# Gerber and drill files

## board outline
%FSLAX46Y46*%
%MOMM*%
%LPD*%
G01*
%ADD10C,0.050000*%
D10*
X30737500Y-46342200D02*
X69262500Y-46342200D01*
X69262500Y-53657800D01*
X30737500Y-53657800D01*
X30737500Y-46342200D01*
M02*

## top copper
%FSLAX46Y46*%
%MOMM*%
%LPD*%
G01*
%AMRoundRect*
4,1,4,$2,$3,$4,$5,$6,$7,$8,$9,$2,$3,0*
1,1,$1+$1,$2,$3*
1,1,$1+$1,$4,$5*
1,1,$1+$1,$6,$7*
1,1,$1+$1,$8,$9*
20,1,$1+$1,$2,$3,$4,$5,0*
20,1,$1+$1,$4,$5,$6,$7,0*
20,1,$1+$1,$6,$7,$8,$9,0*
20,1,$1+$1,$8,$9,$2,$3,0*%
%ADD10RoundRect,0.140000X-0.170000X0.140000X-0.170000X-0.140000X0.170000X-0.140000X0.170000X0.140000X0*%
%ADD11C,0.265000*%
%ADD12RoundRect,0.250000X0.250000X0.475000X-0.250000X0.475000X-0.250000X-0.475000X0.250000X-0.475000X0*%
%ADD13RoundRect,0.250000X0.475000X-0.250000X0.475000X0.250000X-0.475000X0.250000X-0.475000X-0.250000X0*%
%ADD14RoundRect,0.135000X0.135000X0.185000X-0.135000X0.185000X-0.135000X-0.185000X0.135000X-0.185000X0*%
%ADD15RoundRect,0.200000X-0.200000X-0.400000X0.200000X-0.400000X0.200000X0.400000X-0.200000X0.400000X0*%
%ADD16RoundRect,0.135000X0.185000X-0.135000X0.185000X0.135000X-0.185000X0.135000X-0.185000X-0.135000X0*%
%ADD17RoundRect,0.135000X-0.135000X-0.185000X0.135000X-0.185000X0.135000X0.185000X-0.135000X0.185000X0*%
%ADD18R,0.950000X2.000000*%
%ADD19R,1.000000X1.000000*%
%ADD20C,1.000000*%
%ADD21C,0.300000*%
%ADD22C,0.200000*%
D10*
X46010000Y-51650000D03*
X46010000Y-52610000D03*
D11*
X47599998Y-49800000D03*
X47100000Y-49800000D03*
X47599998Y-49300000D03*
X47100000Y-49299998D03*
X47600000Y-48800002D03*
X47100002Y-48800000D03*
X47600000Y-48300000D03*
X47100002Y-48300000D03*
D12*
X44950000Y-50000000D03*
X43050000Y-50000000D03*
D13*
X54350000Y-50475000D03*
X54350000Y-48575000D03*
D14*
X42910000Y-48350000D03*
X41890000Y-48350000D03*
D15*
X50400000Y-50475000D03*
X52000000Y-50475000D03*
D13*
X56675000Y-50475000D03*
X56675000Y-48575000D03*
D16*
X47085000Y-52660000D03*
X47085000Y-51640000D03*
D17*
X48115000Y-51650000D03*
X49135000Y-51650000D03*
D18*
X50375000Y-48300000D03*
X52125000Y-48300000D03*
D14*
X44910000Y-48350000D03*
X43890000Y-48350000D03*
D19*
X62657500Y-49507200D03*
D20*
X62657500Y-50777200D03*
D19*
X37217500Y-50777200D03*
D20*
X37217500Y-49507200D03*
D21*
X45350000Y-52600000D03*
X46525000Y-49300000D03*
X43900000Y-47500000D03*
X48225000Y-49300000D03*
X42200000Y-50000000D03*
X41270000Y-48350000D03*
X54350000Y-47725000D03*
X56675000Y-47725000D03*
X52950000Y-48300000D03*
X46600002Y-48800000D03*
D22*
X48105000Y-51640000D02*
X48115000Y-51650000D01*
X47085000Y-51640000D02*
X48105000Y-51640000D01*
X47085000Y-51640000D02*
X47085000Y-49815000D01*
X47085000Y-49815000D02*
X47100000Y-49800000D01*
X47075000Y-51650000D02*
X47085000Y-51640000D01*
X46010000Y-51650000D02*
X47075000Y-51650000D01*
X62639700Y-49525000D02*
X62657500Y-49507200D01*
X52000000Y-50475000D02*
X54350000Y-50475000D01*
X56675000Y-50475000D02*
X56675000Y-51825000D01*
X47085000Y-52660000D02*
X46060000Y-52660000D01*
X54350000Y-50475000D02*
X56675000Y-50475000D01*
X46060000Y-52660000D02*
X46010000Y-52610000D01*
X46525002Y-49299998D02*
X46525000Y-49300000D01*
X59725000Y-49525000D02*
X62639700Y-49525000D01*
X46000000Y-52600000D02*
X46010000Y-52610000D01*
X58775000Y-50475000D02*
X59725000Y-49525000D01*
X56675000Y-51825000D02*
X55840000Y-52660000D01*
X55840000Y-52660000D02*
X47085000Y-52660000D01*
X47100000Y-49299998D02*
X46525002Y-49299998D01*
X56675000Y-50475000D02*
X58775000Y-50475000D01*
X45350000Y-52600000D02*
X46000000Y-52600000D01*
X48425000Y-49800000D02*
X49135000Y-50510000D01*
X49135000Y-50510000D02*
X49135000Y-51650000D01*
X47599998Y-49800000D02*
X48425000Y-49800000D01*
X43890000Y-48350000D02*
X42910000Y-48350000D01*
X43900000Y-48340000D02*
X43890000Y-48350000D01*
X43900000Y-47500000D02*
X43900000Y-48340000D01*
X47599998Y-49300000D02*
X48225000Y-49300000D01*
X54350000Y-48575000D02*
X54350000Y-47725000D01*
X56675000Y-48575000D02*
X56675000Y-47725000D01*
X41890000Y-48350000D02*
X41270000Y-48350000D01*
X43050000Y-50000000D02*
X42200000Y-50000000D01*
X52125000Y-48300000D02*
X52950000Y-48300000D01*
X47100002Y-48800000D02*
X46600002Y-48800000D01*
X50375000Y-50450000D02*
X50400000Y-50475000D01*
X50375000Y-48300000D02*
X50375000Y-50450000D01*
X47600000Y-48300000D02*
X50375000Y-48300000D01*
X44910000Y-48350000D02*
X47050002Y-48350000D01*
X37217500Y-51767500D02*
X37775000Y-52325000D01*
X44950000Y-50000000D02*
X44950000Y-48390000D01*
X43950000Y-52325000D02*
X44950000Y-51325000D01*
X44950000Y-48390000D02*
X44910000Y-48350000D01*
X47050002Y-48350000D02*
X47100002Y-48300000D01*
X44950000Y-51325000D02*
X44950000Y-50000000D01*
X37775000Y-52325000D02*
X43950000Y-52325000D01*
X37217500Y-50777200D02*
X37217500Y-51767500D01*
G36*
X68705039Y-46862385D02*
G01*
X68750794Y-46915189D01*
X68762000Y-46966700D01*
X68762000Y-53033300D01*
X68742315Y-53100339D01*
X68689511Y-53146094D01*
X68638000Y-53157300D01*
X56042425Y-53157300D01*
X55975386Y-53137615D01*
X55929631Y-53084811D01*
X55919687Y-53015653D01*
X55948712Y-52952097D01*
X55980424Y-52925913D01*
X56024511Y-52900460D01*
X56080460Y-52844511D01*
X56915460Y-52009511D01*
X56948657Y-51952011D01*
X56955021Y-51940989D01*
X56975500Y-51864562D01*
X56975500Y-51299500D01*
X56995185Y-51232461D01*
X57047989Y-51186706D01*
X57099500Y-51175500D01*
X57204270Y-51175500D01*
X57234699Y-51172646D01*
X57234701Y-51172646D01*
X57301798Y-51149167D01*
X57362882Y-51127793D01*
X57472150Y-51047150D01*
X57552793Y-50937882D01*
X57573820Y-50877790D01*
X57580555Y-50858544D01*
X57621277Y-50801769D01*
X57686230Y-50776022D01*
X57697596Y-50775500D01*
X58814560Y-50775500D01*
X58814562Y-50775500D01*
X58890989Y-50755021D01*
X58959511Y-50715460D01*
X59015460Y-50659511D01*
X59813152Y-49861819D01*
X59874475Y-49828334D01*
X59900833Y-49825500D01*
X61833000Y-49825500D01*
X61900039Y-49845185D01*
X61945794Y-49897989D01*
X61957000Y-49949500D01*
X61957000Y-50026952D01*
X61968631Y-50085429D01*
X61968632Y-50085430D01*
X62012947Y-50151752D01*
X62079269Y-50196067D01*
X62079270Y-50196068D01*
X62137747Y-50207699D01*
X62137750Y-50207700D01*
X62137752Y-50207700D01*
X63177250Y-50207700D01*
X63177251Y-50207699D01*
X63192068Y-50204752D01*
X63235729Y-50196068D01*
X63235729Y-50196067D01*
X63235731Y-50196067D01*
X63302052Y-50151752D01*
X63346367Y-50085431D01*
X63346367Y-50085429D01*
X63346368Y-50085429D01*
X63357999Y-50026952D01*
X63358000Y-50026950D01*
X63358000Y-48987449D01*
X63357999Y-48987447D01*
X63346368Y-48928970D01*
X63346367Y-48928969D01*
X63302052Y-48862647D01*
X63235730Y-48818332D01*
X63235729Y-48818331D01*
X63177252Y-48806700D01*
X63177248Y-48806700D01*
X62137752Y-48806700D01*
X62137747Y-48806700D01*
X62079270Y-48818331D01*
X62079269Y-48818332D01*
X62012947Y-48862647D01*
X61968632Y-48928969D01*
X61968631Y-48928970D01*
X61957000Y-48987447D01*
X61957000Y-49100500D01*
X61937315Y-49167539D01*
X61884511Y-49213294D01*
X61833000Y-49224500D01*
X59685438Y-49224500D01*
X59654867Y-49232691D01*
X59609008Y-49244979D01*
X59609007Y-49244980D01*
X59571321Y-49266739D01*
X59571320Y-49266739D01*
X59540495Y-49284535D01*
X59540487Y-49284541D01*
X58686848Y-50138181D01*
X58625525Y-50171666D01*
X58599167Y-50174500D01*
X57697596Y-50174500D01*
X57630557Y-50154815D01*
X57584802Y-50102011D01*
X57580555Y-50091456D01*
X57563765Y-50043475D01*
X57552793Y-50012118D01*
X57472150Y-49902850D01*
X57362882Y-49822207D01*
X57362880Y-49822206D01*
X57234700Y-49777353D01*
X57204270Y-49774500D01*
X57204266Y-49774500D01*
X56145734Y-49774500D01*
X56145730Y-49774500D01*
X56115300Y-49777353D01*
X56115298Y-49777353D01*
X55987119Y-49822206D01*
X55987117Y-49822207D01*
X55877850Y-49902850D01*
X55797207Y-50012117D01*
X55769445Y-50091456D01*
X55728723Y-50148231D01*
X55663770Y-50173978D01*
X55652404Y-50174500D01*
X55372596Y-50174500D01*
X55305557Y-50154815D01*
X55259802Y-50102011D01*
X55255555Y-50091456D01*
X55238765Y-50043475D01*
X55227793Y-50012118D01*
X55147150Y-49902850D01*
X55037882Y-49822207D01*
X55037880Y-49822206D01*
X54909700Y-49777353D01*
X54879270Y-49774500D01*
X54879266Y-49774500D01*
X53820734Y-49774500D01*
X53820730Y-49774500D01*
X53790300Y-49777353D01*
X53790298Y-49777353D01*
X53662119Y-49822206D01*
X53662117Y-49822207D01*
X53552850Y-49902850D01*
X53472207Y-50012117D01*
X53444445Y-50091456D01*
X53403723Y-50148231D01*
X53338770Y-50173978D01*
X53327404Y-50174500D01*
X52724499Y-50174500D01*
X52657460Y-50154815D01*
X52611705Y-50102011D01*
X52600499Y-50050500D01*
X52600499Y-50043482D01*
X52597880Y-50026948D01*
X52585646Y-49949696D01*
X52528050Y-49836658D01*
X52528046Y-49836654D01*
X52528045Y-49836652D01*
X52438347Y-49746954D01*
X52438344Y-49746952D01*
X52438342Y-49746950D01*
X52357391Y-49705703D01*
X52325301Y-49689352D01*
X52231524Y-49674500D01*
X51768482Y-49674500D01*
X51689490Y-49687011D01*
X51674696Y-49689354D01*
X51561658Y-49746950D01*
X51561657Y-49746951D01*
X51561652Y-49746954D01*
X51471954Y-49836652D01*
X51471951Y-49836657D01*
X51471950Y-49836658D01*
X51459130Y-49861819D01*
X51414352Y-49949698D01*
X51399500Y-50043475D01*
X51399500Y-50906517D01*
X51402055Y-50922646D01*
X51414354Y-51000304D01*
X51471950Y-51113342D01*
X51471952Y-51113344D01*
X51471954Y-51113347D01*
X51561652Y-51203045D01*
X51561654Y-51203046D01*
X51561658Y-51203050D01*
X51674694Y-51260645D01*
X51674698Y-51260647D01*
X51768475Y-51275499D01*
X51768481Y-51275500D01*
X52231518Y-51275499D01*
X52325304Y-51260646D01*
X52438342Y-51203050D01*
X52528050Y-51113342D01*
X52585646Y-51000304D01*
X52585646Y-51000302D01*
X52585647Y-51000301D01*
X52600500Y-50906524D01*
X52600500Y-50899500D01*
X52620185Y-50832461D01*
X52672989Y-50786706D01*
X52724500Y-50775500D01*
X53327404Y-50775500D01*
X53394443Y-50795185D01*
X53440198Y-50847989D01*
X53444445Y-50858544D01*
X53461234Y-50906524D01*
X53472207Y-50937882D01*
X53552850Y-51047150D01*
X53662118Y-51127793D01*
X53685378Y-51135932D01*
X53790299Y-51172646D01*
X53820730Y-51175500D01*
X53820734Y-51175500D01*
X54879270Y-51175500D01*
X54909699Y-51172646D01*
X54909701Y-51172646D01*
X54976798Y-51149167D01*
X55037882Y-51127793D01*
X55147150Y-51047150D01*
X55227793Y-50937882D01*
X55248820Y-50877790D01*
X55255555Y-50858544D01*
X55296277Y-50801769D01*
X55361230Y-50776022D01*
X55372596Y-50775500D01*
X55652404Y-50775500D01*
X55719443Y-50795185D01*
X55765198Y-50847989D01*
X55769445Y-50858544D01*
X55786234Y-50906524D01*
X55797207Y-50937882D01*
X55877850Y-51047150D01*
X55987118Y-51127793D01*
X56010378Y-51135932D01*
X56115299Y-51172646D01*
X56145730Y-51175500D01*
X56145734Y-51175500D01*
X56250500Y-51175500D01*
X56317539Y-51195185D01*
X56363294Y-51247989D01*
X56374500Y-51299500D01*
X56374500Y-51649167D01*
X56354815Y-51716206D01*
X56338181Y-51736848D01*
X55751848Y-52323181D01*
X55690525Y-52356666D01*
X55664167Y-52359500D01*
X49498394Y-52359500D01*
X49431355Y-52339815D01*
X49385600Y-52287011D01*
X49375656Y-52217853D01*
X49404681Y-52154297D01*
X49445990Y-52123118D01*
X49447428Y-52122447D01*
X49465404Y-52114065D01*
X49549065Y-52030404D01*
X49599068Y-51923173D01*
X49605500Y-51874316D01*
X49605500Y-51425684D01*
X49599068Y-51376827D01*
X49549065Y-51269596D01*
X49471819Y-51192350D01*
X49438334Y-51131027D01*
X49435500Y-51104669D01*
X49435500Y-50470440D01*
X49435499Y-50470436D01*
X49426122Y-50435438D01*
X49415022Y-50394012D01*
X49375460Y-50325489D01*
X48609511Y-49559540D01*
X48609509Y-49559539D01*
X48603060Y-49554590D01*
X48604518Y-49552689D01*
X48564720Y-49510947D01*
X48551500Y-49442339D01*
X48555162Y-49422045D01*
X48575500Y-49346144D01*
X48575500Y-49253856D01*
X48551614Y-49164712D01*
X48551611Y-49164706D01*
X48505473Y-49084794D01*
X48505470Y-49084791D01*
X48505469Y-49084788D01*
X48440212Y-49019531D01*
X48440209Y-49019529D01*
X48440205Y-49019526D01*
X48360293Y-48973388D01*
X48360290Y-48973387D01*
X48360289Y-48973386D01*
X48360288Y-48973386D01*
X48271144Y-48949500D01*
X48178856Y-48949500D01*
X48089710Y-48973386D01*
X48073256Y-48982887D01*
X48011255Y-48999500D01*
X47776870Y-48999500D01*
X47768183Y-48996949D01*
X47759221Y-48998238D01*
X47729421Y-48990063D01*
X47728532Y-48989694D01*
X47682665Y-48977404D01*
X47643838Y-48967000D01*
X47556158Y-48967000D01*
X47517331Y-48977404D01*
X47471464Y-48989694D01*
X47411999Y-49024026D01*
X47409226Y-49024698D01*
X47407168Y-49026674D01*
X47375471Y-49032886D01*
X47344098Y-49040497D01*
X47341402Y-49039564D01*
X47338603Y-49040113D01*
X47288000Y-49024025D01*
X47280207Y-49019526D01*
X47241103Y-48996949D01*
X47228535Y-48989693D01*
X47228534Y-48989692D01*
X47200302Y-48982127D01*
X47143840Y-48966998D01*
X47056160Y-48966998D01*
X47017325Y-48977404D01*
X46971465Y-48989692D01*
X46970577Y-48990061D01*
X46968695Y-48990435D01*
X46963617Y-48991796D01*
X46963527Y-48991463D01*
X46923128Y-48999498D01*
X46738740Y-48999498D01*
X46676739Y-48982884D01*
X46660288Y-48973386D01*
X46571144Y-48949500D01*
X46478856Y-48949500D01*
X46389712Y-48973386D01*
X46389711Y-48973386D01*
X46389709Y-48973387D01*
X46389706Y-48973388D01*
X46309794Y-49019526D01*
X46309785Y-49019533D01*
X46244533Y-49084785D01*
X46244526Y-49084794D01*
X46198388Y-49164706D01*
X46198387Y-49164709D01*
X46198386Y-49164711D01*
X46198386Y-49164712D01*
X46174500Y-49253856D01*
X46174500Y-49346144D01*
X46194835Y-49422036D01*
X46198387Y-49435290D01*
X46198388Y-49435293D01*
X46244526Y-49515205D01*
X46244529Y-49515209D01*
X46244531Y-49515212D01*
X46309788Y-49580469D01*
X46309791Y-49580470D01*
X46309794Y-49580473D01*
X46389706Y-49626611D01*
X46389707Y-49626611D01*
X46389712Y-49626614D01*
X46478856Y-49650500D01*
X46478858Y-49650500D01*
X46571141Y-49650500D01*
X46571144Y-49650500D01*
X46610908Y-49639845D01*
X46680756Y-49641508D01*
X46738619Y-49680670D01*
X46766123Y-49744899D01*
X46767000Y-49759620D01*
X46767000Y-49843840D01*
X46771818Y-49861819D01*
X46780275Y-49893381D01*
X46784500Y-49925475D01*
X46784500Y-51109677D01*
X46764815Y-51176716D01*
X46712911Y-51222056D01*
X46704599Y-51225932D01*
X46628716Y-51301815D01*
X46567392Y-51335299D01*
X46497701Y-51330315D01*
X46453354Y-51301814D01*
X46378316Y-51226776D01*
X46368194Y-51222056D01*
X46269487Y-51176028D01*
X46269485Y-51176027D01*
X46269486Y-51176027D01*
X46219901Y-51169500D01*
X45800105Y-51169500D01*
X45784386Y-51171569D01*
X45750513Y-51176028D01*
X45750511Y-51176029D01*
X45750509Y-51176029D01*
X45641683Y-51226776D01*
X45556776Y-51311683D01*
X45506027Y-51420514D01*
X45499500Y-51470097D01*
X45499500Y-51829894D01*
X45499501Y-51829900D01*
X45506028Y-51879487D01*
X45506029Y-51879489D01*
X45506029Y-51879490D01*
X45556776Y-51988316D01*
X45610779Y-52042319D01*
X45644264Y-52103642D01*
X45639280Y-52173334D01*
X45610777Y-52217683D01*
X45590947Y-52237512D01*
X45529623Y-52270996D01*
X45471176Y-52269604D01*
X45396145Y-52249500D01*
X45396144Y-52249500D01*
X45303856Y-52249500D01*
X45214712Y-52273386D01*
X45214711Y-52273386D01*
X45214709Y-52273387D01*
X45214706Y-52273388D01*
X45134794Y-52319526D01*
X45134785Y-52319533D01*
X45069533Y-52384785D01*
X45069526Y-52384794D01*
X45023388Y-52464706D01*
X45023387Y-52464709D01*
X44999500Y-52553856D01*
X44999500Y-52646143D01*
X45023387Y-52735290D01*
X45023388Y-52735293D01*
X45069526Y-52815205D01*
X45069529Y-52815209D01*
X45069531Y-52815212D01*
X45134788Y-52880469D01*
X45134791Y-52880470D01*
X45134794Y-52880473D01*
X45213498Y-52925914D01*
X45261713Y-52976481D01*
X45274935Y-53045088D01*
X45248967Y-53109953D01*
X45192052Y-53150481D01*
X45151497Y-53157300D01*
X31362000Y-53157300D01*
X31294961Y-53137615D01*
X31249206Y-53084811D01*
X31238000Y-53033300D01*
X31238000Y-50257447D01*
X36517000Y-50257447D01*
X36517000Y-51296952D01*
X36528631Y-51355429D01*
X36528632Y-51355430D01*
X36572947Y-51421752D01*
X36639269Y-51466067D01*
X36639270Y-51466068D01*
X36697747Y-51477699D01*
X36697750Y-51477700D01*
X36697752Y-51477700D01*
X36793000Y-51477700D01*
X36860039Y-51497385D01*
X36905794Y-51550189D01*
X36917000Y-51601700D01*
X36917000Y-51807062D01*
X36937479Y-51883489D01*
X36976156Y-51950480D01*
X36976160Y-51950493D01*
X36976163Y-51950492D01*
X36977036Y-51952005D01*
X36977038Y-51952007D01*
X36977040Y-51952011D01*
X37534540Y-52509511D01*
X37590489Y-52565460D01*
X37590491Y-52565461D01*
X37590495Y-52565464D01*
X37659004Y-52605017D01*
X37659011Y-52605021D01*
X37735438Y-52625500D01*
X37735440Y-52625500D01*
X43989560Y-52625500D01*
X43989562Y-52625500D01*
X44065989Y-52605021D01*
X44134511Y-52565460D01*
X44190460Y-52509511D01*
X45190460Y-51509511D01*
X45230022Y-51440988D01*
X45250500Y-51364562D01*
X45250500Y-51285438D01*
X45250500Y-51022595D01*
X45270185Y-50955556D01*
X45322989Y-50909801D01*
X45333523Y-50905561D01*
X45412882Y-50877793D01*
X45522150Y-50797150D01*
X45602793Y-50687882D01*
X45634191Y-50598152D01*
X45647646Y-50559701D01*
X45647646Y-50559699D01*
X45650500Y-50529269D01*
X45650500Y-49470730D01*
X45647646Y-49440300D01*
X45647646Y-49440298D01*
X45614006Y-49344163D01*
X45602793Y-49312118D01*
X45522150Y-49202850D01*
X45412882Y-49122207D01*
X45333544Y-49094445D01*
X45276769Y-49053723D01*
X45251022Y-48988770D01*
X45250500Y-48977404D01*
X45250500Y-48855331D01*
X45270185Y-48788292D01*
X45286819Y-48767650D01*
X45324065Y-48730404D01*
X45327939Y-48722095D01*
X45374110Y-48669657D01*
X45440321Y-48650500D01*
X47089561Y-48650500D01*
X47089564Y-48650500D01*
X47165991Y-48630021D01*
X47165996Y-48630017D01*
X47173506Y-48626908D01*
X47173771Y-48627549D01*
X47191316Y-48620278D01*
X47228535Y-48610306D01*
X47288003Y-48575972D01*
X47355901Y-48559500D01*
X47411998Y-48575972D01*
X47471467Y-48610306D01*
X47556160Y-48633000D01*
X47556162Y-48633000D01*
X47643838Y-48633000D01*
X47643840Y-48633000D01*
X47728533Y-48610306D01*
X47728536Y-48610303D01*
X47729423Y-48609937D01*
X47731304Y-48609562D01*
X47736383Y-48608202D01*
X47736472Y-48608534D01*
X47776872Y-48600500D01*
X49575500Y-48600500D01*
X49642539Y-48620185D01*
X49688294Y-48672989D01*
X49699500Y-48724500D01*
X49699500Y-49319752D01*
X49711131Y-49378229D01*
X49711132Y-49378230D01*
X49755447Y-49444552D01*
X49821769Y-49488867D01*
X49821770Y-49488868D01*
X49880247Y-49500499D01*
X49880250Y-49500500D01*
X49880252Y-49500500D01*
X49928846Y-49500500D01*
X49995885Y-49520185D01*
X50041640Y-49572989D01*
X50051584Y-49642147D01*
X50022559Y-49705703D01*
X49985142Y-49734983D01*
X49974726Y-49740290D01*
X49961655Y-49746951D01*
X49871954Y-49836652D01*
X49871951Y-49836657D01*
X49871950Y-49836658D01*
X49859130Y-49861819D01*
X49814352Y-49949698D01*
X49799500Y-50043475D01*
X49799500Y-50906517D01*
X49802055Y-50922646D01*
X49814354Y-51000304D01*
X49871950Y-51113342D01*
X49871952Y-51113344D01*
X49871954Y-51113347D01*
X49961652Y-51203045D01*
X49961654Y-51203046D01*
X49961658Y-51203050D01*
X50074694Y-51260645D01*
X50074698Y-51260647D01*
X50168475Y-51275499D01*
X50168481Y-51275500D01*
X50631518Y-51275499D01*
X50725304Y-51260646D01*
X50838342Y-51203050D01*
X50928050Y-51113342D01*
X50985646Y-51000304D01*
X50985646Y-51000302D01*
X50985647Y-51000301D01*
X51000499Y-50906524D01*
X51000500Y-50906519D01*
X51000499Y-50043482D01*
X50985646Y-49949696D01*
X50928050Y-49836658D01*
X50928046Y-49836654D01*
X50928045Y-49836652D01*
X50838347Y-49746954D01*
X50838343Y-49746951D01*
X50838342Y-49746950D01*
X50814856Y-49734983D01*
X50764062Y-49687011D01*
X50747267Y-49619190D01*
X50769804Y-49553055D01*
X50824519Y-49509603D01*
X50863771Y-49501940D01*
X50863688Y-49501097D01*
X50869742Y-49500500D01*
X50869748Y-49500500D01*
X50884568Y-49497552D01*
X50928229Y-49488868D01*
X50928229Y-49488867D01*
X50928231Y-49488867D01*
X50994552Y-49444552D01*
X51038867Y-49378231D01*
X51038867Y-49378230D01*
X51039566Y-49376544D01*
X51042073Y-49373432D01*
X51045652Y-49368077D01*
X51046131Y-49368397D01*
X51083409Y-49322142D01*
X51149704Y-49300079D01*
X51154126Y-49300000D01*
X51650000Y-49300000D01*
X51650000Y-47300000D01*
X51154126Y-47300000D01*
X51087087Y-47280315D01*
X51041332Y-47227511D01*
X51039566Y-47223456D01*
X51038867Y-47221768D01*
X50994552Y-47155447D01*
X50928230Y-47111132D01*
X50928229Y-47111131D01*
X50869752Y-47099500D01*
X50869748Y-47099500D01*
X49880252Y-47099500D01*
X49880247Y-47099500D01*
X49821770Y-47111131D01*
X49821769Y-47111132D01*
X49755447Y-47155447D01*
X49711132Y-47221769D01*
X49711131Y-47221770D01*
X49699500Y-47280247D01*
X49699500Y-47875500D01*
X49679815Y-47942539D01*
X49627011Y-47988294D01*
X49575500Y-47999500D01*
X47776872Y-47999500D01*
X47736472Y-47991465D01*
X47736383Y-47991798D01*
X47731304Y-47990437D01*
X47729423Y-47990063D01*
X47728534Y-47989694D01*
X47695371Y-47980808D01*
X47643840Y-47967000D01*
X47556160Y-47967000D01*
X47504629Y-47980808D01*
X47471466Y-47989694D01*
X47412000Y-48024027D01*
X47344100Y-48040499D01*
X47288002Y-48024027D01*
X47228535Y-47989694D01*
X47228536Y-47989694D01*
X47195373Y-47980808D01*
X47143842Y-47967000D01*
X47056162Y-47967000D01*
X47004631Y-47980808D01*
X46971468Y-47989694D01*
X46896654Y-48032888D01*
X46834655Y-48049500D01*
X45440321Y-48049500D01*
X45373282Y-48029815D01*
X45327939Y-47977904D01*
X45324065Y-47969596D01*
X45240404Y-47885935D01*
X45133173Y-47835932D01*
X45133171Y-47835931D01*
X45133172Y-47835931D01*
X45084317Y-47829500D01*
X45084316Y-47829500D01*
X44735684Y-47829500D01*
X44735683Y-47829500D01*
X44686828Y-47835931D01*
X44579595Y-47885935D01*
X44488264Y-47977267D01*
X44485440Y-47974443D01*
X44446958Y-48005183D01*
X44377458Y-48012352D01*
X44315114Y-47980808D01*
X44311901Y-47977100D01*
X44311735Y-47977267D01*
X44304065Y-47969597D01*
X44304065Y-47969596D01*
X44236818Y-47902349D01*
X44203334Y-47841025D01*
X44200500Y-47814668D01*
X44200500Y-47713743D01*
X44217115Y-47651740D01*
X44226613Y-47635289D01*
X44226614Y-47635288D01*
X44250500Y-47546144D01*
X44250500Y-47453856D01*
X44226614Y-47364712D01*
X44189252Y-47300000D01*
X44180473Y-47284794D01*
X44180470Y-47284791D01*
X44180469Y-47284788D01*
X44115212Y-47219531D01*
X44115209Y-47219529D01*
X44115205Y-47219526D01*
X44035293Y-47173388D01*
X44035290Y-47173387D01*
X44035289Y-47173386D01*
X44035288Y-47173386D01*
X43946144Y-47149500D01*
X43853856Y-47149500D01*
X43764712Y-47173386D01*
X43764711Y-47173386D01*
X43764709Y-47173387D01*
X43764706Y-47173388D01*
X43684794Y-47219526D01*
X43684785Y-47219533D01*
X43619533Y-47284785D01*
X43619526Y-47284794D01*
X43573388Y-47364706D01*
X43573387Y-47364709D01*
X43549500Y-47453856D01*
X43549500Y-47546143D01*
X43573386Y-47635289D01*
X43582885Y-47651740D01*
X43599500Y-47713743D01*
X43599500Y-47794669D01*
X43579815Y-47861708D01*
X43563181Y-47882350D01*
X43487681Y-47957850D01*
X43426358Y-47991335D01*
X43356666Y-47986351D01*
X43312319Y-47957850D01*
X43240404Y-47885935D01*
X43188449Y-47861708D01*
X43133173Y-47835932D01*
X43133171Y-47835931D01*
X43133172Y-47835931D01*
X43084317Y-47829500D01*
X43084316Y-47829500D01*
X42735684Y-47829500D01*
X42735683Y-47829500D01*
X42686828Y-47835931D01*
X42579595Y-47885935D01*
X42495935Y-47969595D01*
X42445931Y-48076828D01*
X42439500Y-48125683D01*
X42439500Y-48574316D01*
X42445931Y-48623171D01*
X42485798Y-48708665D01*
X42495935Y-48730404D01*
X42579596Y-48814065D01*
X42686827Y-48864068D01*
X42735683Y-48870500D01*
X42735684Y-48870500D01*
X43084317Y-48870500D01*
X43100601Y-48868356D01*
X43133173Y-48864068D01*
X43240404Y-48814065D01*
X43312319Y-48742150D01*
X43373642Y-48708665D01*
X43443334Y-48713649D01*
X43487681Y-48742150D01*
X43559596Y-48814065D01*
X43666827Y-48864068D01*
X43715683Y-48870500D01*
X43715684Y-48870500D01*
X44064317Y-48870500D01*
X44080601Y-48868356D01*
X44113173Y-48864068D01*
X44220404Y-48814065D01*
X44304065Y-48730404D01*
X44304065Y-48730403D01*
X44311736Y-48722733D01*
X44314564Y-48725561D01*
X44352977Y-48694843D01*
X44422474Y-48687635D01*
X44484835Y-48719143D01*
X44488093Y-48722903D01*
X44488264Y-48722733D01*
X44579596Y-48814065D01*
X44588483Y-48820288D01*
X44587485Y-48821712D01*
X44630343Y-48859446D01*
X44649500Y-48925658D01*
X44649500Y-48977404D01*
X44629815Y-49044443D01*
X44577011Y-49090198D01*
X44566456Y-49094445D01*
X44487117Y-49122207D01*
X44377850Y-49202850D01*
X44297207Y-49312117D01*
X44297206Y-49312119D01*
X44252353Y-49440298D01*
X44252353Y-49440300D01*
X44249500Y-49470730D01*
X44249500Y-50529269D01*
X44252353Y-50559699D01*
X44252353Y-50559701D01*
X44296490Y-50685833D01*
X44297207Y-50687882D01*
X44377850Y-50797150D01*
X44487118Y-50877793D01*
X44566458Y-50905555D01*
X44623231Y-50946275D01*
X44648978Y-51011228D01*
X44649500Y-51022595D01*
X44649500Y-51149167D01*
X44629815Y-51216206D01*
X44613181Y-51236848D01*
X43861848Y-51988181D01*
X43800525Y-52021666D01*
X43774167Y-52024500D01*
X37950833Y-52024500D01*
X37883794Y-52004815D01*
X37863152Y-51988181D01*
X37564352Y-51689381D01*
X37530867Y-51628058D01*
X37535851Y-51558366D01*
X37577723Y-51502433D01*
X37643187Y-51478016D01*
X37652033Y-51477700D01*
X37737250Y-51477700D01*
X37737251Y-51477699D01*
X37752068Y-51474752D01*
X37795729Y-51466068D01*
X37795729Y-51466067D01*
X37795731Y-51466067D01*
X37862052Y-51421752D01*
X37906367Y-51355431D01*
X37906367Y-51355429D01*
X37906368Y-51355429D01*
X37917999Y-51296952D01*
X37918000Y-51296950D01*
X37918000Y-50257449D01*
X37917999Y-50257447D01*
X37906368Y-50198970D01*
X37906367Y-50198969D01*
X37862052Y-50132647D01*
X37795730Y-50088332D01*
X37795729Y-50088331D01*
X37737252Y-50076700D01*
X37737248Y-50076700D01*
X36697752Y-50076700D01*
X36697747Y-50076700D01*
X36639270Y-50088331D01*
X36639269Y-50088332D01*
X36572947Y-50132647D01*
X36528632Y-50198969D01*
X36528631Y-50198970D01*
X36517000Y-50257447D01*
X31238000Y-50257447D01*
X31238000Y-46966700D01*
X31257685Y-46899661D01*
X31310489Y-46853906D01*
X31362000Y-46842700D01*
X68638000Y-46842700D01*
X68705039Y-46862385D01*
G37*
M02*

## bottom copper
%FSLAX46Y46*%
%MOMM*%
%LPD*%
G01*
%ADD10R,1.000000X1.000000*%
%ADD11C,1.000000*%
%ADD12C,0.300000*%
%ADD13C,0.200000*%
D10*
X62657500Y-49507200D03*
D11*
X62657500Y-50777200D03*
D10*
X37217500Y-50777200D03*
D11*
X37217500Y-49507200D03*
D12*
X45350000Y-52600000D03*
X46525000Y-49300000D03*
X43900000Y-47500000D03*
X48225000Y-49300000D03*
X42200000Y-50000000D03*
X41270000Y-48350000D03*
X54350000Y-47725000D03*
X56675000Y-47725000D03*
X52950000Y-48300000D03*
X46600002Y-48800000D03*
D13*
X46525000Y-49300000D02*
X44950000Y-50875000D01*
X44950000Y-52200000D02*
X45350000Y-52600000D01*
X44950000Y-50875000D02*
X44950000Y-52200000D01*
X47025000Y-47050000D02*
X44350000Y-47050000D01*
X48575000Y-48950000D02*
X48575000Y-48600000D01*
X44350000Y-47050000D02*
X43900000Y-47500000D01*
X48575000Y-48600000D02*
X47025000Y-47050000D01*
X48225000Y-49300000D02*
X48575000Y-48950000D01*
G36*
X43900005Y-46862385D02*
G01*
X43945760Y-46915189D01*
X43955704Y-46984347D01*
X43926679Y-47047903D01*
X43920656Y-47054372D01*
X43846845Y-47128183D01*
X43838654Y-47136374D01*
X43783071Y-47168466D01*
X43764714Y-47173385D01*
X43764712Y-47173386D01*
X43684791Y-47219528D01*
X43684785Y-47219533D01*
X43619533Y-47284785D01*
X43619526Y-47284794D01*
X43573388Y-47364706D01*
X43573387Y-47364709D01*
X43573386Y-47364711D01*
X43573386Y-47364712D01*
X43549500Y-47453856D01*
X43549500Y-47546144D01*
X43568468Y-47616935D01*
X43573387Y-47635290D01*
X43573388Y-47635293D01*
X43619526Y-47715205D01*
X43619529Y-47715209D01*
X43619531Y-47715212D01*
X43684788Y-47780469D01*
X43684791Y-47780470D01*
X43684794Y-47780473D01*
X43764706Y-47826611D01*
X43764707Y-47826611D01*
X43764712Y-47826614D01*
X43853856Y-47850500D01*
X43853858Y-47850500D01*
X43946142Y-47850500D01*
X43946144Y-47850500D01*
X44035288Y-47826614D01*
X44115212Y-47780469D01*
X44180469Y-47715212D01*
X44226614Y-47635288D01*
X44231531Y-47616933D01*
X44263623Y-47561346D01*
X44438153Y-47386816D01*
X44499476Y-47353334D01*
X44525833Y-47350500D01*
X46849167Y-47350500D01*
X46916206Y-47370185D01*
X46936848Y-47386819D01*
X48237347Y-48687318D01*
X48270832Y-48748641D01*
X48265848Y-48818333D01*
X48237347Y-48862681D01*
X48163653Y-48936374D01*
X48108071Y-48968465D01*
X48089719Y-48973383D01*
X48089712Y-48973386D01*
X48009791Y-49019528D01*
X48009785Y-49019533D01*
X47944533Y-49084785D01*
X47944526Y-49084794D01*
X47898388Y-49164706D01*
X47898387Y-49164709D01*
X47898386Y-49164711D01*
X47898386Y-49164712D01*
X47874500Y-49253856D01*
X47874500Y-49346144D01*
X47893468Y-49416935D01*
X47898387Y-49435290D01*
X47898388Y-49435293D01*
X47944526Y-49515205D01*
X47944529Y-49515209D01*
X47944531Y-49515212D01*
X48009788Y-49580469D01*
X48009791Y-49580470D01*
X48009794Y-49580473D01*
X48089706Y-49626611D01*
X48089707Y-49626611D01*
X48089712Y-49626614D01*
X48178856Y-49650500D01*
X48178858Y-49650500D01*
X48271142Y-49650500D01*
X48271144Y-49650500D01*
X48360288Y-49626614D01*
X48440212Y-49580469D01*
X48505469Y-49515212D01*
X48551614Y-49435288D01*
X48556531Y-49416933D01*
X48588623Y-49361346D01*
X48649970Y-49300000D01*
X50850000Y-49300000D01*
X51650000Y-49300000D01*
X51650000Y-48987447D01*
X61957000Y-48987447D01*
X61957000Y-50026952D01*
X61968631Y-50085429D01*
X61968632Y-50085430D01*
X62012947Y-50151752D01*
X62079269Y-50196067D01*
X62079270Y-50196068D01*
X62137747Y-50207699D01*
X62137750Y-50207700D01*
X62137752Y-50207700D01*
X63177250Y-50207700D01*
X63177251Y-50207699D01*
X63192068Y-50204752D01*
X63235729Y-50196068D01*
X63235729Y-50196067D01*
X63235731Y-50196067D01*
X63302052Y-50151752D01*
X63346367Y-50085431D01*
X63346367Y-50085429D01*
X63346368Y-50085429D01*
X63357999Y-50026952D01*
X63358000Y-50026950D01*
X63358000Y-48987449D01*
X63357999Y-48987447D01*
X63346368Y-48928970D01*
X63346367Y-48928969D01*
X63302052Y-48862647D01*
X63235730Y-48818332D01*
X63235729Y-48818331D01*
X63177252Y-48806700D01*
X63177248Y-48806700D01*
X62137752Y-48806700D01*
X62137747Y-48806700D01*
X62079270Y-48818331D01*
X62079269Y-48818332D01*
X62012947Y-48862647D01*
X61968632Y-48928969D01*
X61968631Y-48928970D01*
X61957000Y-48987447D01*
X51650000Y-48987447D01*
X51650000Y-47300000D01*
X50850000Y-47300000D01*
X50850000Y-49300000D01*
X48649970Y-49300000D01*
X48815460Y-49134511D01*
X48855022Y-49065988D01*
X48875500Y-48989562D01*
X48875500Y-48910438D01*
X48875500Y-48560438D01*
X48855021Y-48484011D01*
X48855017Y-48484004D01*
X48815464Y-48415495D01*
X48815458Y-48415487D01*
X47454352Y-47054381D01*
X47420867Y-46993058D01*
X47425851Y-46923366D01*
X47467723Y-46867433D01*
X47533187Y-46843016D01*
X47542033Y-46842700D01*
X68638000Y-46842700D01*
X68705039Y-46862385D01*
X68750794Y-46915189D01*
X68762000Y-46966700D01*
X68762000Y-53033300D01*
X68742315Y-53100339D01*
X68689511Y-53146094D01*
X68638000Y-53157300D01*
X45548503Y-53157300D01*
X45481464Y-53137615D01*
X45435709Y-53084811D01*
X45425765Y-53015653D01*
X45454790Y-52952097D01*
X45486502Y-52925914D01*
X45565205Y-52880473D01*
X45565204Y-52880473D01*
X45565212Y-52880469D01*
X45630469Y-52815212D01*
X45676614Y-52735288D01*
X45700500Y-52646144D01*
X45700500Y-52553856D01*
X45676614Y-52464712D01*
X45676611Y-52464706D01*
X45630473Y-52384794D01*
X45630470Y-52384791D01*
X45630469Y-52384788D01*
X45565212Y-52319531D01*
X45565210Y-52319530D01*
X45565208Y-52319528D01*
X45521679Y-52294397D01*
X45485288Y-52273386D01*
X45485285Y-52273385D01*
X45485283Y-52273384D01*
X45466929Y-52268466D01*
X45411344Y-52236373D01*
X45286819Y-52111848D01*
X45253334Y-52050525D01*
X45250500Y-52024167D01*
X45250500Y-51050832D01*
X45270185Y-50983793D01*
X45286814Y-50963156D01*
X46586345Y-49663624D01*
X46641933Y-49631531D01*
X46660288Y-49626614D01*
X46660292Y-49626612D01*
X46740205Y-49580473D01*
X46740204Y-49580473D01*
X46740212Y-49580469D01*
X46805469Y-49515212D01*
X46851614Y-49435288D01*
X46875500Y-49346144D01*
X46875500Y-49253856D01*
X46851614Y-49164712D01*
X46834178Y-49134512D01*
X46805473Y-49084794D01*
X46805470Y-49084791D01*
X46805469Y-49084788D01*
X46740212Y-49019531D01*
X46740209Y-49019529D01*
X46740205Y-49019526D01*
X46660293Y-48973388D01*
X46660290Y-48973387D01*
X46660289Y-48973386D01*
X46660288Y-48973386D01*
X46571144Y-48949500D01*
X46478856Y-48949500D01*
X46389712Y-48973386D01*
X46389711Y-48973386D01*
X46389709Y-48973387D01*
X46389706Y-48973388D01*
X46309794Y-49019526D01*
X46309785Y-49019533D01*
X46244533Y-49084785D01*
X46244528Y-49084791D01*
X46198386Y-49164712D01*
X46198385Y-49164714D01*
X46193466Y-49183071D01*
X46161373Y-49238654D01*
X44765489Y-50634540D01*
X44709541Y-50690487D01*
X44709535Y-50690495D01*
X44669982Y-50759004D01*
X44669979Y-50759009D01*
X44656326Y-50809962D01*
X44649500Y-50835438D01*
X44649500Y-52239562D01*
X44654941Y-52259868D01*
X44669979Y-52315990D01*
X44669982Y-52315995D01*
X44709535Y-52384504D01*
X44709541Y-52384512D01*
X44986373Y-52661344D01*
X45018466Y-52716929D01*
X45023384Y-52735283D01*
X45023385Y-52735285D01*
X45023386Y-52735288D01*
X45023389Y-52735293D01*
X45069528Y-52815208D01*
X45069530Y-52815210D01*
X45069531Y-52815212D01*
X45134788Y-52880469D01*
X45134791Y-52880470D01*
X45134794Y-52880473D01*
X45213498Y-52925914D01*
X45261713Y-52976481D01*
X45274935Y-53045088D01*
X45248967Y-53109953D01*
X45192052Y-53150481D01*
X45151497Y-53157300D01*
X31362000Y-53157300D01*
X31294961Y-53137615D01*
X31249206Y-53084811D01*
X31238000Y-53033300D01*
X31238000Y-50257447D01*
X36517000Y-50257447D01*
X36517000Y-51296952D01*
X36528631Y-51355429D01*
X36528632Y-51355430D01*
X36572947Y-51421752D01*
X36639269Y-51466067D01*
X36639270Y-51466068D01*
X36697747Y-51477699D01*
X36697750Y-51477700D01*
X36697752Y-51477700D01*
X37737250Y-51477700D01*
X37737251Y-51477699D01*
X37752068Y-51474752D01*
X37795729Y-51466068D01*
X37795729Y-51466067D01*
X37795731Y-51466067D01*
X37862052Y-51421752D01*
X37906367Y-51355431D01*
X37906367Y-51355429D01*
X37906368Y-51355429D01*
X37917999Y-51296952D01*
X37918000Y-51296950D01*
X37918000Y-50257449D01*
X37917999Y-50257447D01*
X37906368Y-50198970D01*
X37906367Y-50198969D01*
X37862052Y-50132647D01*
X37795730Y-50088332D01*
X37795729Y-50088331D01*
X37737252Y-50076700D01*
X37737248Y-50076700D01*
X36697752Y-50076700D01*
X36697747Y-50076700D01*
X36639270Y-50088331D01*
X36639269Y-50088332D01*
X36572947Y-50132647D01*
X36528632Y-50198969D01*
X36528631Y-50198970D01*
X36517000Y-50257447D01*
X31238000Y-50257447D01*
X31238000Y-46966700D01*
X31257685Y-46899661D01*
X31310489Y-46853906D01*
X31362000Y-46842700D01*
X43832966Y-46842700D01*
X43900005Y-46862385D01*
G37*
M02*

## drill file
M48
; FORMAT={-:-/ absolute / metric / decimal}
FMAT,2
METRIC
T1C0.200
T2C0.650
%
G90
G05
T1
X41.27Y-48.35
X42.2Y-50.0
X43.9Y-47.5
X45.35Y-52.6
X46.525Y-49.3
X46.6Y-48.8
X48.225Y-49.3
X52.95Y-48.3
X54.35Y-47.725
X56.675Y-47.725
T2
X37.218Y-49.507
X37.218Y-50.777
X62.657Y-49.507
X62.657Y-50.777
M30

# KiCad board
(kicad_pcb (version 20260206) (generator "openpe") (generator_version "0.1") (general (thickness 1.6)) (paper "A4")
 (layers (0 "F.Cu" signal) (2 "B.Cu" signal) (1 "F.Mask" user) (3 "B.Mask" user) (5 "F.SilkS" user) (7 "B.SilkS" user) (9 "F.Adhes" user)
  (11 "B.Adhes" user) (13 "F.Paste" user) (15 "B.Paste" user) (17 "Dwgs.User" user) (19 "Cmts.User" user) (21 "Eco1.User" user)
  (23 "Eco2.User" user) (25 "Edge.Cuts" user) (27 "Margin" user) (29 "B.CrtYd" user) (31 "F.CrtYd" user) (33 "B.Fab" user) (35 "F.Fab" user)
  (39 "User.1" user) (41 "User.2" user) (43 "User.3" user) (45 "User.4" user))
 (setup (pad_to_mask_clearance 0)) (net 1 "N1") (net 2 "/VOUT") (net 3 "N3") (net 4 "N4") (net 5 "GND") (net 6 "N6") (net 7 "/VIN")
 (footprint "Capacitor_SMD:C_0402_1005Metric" (layer "F.Cu") (at 46.01 52.13 -90)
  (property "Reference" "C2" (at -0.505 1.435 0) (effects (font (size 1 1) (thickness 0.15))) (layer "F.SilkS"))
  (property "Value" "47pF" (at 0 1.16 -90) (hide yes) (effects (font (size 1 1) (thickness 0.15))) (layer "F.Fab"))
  (pad "1" smd roundrect (at -0.48 0 -90) (size 0.56 0.62) (layers "F.Cu" "F.Mask" "F.Paste") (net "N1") (roundrect_rratio 0.25))
  (pad "2" smd roundrect (at 0.48 0 -90) (size 0.56 0.62) (layers "F.Cu" "F.Mask" "F.Paste") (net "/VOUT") (roundrect_rratio 0.25)))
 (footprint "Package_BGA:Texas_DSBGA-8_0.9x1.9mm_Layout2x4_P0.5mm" (layer "F.Cu") (at 47.35 49.05 180)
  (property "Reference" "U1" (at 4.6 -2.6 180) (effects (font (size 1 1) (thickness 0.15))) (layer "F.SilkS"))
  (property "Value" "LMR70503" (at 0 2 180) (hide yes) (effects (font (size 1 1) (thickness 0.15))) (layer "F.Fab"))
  (pad "" smd rect (at -0.25 0.249998 180) (size 0.3 0.3) (layers "F.Paste") (solder_mask_margin 0.05))
  (pad "" smd rect (at -0.25 0.75 180) (size 0.3 0.3) (layers "F.Paste") (solder_mask_margin 0.05))
  (pad "" smd rect (at -0.249998 -0.75 180) (size 0.3 0.3) (layers "F.Paste") (solder_mask_margin 0.05))
  (pad "" smd rect (at -0.249998 -0.25 180) (size 0.3 0.3) (layers "F.Paste") (solder_mask_margin 0.05))
  (pad "" smd rect (at 0.249998 0.25 180) (size 0.3 0.3) (layers "F.Paste") (solder_mask_margin 0.05))
  (pad "" smd rect (at 0.249998 0.75 180) (size 0.3 0.3) (layers "F.Paste") (solder_mask_margin 0.05))
  (pad "" smd rect (at 0.25 -0.75 180) (size 0.3 0.3) (layers "F.Paste") (solder_mask_margin 0.05))
  (pad "" smd rect (at 0.25 -0.249998 180) (size 0.3 0.3) (layers "F.Paste") (solder_mask_margin 0.05))
  (pad "A1" smd circle (at -0.249998 -0.75 180) (size 0.265 0.265) (layers "F.Cu" "F.Mask") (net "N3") (solder_mask_margin 0.05))
  (pad "A2" smd circle (at 0.25 -0.75 180) (size 0.265 0.265) (layers "F.Cu" "F.Mask") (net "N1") (solder_mask_margin 0.05))
  (pad "B1" smd circle (at -0.249998 -0.25 180) (size 0.265 0.265) (layers "F.Cu" "F.Mask") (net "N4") (solder_mask_margin 0.05))
  (pad "B2" smd circle (at 0.25 -0.249998 180) (size 0.265 0.265) (layers "F.Cu" "F.Mask") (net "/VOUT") (solder_mask_margin 0.05))
  (pad "C1" smd circle (at -0.25 0.249998 180) (size 0.265 0.265) (layers "F.Cu" "F.Mask") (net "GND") (solder_mask_margin 0.05))
  (pad "C2" smd circle (at 0.249998 0.25 180) (size 0.265 0.265) (layers "F.Cu" "F.Mask") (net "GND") (solder_mask_margin 0.05))
  (pad "D1" smd circle (at -0.25 0.75 180) (size 0.265 0.265) (layers "F.Cu" "F.Mask") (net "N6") (solder_mask_margin 0.05))
  (pad "D2" smd circle (at 0.249998 0.75 180) (size 0.265 0.265) (layers "F.Cu" "F.Mask") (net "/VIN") (solder_mask_margin 0.05)))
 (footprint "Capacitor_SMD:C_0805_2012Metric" (layer "F.Cu") (at 44 50 180)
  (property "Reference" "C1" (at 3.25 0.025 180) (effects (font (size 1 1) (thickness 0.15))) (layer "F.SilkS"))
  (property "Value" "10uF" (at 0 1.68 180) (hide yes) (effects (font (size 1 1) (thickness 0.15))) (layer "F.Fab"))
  (pad "1" smd roundrect (at -0.95 0 180) (size 1 1.45) (layers "F.Cu" "F.Mask" "F.Paste") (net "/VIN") (roundrect_rratio 0.25))
  (pad "2" smd roundrect (at 0.95 0 180) (size 1 1.45) (layers "F.Cu" "F.Mask" "F.Paste") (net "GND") (roundrect_rratio 0.25)))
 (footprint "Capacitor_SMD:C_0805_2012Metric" (layer "F.Cu") (at 54.35 49.525 90)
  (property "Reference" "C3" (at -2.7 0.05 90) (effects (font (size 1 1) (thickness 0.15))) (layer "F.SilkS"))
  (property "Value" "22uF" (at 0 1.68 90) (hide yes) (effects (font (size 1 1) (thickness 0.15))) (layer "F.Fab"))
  (pad "1" smd roundrect (at -0.95 0 90) (size 1 1.45) (layers "F.Cu" "F.Mask" "F.Paste") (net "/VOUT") (roundrect_rratio 0.25))
  (pad "2" smd roundrect (at 0.95 0 90) (size 1 1.45) (layers "F.Cu" "F.Mask" "F.Paste") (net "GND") (roundrect_rratio 0.25)))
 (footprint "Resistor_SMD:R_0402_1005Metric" (layer "F.Cu") (at 42.4 48.35 180)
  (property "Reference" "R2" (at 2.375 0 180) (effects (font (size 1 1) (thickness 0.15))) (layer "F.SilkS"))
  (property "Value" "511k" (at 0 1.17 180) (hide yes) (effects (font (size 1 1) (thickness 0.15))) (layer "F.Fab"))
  (pad "1" smd roundrect (at -0.51 0 180) (size 0.54 0.64) (layers "F.Cu" "F.Mask" "F.Paste") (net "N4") (roundrect_rratio 0.25))
  (pad "2" smd roundrect (at 0.51 0 180) (size 0.54 0.64) (layers "F.Cu" "F.Mask" "F.Paste") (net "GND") (roundrect_rratio 0.25)))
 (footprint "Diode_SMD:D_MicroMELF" (layer "F.Cu") (at 51.2 50.475 0)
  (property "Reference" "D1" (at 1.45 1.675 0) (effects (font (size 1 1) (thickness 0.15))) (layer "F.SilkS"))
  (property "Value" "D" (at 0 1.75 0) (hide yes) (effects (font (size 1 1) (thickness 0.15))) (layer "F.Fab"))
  (pad "1" smd roundrect (at -0.8 0 0) (size 0.8 1.2) (layers "F.Cu" "F.Mask" "F.Paste") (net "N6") (roundrect_rratio 0.25))
  (pad "2" smd roundrect (at 0.8 0 0) (size 0.8 1.2) (layers "F.Cu" "F.Mask" "F.Paste") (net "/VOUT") (roundrect_rratio 0.25)))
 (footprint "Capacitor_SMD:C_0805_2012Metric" (layer "F.Cu") (at 56.675 49.525 90)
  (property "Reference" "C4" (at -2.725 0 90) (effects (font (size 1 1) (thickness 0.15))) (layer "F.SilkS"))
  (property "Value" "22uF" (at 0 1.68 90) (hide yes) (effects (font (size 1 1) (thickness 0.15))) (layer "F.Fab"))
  (pad "1" smd roundrect (at -0.95 0 90) (size 1 1.45) (layers "F.Cu" "F.Mask" "F.Paste") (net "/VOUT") (roundrect_rratio 0.25))
  (pad "2" smd roundrect (at 0.95 0 90) (size 1 1.45) (layers "F.Cu" "F.Mask" "F.Paste") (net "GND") (roundrect_rratio 0.25)))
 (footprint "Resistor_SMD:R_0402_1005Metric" (layer "F.Cu") (at 47.085 52.15 90)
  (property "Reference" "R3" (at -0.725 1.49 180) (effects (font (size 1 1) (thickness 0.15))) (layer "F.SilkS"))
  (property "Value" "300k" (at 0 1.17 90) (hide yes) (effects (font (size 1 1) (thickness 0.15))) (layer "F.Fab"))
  (pad "1" smd roundrect (at -0.51 0 90) (size 0.54 0.64) (layers "F.Cu" "F.Mask" "F.Paste") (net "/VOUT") (roundrect_rratio 0.25))
  (pad "2" smd roundrect (at 0.51 0 90) (size 0.54 0.64) (layers "F.Cu" "F.Mask" "F.Paste") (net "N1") (roundrect_rratio 0.25)))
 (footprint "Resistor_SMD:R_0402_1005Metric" (layer "F.Cu") (at 48.625 51.65 0)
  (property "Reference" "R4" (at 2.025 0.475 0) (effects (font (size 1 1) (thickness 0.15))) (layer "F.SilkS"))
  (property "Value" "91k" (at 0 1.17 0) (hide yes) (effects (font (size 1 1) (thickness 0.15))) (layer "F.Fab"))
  (pad "1" smd roundrect (at -0.51 0 0) (size 0.54 0.64) (layers "F.Cu" "F.Mask" "F.Paste") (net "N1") (roundrect_rratio 0.25))
  (pad "2" smd roundrect (at 0.51 0 0) (size 0.54 0.64) (layers "F.Cu" "F.Mask" "F.Paste") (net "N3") (roundrect_rratio 0.25)))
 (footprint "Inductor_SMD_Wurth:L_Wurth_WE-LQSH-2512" (layer "F.Cu") (at 51.25 48.3 0)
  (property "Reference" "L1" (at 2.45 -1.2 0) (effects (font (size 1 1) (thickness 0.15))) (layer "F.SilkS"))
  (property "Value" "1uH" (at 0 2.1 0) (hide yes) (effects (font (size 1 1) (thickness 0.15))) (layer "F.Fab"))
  (pad "1" smd rect (at -0.875 0 0) (size 0.95 2) (layers "F.Cu" "F.Mask" "F.Paste") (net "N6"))
  (pad "2" smd rect (at 0.875 0 0) (size 0.95 2) (layers "F.Cu" "F.Mask" "F.Paste") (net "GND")))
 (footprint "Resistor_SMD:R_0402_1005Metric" (layer "F.Cu") (at 44.4 48.35 180)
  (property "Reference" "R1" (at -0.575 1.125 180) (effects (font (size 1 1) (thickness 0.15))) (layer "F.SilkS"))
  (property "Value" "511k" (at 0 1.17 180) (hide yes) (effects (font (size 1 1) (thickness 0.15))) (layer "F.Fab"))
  (pad "1" smd roundrect (at -0.51 0 180) (size 0.54 0.64) (layers "F.Cu" "F.Mask" "F.Paste") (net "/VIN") (roundrect_rratio 0.25))
  (pad "2" smd roundrect (at 0.51 0 180) (size 0.54 0.64) (layers "F.Cu" "F.Mask" "F.Paste") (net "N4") (roundrect_rratio 0.25)))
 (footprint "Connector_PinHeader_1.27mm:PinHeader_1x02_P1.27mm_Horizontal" (layer "F.Cu") (at 65.0875 50.1422 0)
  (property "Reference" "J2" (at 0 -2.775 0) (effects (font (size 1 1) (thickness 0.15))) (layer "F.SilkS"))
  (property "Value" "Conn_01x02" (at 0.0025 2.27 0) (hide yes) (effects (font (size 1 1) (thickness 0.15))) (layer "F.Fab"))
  (pad "1" thru_hole rect (at -2.43 -0.635 0) (size 1 1) (drill 0.65) (layers "*.Cu" "*.Mask") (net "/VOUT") (remove_unused_layers no))
  (pad "2" thru_hole circle (at -2.43 0.635 0) (size 1 1) (drill 0.65) (layers "*.Cu" "*.Mask") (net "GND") (remove_unused_layers no)))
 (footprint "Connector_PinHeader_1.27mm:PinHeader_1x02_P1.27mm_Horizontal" (layer "F.Cu") (at 34.7875 50.1422 180)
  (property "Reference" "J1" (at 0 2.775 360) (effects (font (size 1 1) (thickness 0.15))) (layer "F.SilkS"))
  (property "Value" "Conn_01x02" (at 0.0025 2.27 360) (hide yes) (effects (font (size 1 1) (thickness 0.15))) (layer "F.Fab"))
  (pad "1" thru_hole rect (at -2.43 -0.635 180) (size 1 1) (drill 0.65) (layers "*.Cu" "*.Mask") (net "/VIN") (remove_unused_layers no))
  (pad "2" thru_hole circle (at -2.43 0.635 180) (size 1 1) (drill 0.65) (layers "*.Cu" "*.Mask") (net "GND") (remove_unused_layers no)))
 (gr_poly
  (pts (xy 30.7375 46.3422) (xy 69.2625 46.3422) (xy 69.2625 53.6578) (xy 30.7375 53.6578)) (stroke (width 0.05) (type solid)) (fill no)
  (layer "Edge.Cuts"))
 (segment (start 48.105 51.64) (end 48.115 51.65) (width 0.2) (layer "F.Cu") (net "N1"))
 (segment (start 47.085 51.64) (end 48.105 51.64) (width 0.2) (layer "F.Cu") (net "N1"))
 (segment (start 47.085 51.64) (end 47.085 49.815) (width 0.2) (layer "F.Cu") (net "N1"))
 (segment (start 47.085 49.815) (end 47.1 49.8) (width 0.2) (layer "F.Cu") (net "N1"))
 (segment (start 47.075 51.65) (end 47.085 51.64) (width 0.2) (layer "F.Cu") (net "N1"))
 (segment (start 46.01 51.65) (end 47.075 51.65) (width 0.2) (layer "F.Cu") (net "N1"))
 (segment (start 62.6397 49.525) (end 62.6575 49.5072) (width 0.2) (layer "F.Cu") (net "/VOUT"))
 (segment (start 52 50.475) (end 54.35 50.475) (width 0.2) (layer "F.Cu") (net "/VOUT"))
 (segment (start 56.675 50.475) (end 56.675 51.825) (width 0.2) (layer "F.Cu") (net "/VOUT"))
 (segment (start 47.085 52.66) (end 46.06 52.66) (width 0.2) (layer "F.Cu") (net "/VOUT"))
 (segment (start 54.35 50.475) (end 56.675 50.475) (width 0.2) (layer "F.Cu") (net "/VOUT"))
 (segment (start 46.06 52.66) (end 46.01 52.61) (width 0.2) (layer "F.Cu") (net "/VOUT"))
 (segment (start 46.525002 49.299998) (end 46.525 49.3) (width 0.2) (layer "F.Cu") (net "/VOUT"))
 (segment (start 59.725 49.525) (end 62.6397 49.525) (width 0.2) (layer "F.Cu") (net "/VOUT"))
 (segment (start 46 52.6) (end 46.01 52.61) (width 0.2) (layer "F.Cu") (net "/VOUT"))
 (segment (start 58.775 50.475) (end 59.725 49.525) (width 0.2) (layer "F.Cu") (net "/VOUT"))
 (segment (start 56.675 51.825) (end 55.84 52.66) (width 0.2) (layer "F.Cu") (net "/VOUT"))
 (segment (start 55.84 52.66) (end 47.085 52.66) (width 0.2) (layer "F.Cu") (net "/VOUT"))
 (segment (start 47.1 49.299998) (end 46.525002 49.299998) (width 0.2) (layer "F.Cu") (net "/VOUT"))
 (segment (start 56.675 50.475) (end 58.775 50.475) (width 0.2) (layer "F.Cu") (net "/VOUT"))
 (segment (start 45.35 52.6) (end 46 52.6) (width 0.2) (layer "F.Cu") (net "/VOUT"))
 (segment (start 46.525 49.3) (end 44.95 50.875) (width 0.2) (layer "B.Cu") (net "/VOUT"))
 (segment (start 44.95 52.2) (end 45.35 52.6) (width 0.2) (layer "B.Cu") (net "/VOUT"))
 (segment (start 44.95 50.875) (end 44.95 52.2) (width 0.2) (layer "B.Cu") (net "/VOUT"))
 (segment (start 48.425 49.8) (end 49.135 50.51) (width 0.2) (layer "F.Cu") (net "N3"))
 (segment (start 49.135 50.51) (end 49.135 51.65) (width 0.2) (layer "F.Cu") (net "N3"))
 (segment (start 47.599998 49.8) (end 48.425 49.8) (width 0.2) (layer "F.Cu") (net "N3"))
 (segment (start 43.89 48.35) (end 42.91 48.35) (width 0.2) (layer "F.Cu") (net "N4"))
 (segment (start 43.9 48.34) (end 43.89 48.35) (width 0.2) (layer "F.Cu") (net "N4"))
 (segment (start 43.9 47.5) (end 43.9 48.34) (width 0.2) (layer "F.Cu") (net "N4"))
 (segment (start 47.599998 49.3) (end 48.225 49.3) (width 0.2) (layer "F.Cu") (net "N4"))
 (segment (start 47.025 47.05) (end 44.35 47.05) (width 0.2) (layer "B.Cu") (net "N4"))
 (segment (start 48.575 48.95) (end 48.575 48.6) (width 0.2) (layer "B.Cu") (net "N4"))
 (segment (start 44.35 47.05) (end 43.9 47.5) (width 0.2) (layer "B.Cu") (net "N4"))
 (segment (start 48.575 48.6) (end 47.025 47.05) (width 0.2) (layer "B.Cu") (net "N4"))
 (segment (start 48.225 49.3) (end 48.575 48.95) (width 0.2) (layer "B.Cu") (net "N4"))
 (segment (start 54.35 48.575) (end 54.35 47.725) (width 0.2) (layer "F.Cu") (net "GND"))
 (segment (start 56.675 48.575) (end 56.675 47.725) (width 0.2) (layer "F.Cu") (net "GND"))
 (segment (start 41.89 48.35) (end 41.27 48.35) (width 0.2) (layer "F.Cu") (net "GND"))
 (segment (start 43.05 50) (end 42.2 50) (width 0.2) (layer "F.Cu") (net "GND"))
 (segment (start 52.125 48.3) (end 52.95 48.3) (width 0.2) (layer "F.Cu") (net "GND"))
 (segment (start 47.100002 48.8) (end 46.600002 48.8) (width 0.2) (layer "F.Cu") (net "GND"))
 (segment (start 50.375 50.45) (end 50.4 50.475) (width 0.2) (layer "F.Cu") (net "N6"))
 (segment (start 50.375 48.3) (end 50.375 50.45) (width 0.2) (layer "F.Cu") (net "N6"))
 (segment (start 47.6 48.3) (end 50.375 48.3) (width 0.2) (layer "F.Cu") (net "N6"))
 (segment (start 44.91 48.35) (end 47.050002 48.35) (width 0.2) (layer "F.Cu") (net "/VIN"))
 (segment (start 37.2175 51.7675) (end 37.775 52.325) (width 0.2) (layer "F.Cu") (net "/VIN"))
 (segment (start 44.95 50) (end 44.95 48.39) (width 0.2) (layer "F.Cu") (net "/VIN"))
 (segment (start 43.95 52.325) (end 44.95 51.325) (width 0.2) (layer "F.Cu") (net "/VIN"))
 (segment (start 44.95 48.39) (end 44.91 48.35) (width 0.2) (layer "F.Cu") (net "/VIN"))
 (segment (start 47.050002 48.35) (end 47.100002 48.3) (width 0.2) (layer "F.Cu") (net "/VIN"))
 (segment (start 44.95 51.325) (end 44.95 50) (width 0.2) (layer "F.Cu") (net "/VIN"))
 (segment (start 37.775 52.325) (end 43.95 52.325) (width 0.2) (layer "F.Cu") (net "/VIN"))
 (segment (start 37.2175 50.7772) (end 37.2175 51.7675) (width 0.2) (layer "F.Cu") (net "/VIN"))
 (via (at 45.35 52.6) (size 0.3) (drill 0.2) (layers "F.Cu" "B.Cu") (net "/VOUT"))
 (via (at 46.525 49.3) (size 0.3) (drill 0.2) (layers "F.Cu" "B.Cu") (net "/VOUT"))
 (via (at 43.9 47.5) (size 0.3) (drill 0.2) (layers "F.Cu" "B.Cu") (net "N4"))
 (via (at 48.225 49.3) (size 0.3) (drill 0.2) (layers "F.Cu" "B.Cu") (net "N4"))
 (via (at 42.2 50) (size 0.3) (drill 0.2) (layers "F.Cu" "B.Cu") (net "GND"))
 (via (at 41.27 48.35) (size 0.3) (drill 0.2) (layers "F.Cu" "B.Cu") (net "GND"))
 (via (at 54.35 47.725) (size 0.3) (drill 0.2) (layers "F.Cu" "B.Cu") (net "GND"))
 (via (at 56.675 47.725) (size 0.3) (drill 0.2) (layers "F.Cu" "B.Cu") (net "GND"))
 (via (at 52.95 48.3) (size 0.3) (drill 0.2) (layers "F.Cu" "B.Cu") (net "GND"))
 (via (at 46.600002 48.8) (size 0.3) (drill 0.2) (layers "F.Cu" "B.Cu") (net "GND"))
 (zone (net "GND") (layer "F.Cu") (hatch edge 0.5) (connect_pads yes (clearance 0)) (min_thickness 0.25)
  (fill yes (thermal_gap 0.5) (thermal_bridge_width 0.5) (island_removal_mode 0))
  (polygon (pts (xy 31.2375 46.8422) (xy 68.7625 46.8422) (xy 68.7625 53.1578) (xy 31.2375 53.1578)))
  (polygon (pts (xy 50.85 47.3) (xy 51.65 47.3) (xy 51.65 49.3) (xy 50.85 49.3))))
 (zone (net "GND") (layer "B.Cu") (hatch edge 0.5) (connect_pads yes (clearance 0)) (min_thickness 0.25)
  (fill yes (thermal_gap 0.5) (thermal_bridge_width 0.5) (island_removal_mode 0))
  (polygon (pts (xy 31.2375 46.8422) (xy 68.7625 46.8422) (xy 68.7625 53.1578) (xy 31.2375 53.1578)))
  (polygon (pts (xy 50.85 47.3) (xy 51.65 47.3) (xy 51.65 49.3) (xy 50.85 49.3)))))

